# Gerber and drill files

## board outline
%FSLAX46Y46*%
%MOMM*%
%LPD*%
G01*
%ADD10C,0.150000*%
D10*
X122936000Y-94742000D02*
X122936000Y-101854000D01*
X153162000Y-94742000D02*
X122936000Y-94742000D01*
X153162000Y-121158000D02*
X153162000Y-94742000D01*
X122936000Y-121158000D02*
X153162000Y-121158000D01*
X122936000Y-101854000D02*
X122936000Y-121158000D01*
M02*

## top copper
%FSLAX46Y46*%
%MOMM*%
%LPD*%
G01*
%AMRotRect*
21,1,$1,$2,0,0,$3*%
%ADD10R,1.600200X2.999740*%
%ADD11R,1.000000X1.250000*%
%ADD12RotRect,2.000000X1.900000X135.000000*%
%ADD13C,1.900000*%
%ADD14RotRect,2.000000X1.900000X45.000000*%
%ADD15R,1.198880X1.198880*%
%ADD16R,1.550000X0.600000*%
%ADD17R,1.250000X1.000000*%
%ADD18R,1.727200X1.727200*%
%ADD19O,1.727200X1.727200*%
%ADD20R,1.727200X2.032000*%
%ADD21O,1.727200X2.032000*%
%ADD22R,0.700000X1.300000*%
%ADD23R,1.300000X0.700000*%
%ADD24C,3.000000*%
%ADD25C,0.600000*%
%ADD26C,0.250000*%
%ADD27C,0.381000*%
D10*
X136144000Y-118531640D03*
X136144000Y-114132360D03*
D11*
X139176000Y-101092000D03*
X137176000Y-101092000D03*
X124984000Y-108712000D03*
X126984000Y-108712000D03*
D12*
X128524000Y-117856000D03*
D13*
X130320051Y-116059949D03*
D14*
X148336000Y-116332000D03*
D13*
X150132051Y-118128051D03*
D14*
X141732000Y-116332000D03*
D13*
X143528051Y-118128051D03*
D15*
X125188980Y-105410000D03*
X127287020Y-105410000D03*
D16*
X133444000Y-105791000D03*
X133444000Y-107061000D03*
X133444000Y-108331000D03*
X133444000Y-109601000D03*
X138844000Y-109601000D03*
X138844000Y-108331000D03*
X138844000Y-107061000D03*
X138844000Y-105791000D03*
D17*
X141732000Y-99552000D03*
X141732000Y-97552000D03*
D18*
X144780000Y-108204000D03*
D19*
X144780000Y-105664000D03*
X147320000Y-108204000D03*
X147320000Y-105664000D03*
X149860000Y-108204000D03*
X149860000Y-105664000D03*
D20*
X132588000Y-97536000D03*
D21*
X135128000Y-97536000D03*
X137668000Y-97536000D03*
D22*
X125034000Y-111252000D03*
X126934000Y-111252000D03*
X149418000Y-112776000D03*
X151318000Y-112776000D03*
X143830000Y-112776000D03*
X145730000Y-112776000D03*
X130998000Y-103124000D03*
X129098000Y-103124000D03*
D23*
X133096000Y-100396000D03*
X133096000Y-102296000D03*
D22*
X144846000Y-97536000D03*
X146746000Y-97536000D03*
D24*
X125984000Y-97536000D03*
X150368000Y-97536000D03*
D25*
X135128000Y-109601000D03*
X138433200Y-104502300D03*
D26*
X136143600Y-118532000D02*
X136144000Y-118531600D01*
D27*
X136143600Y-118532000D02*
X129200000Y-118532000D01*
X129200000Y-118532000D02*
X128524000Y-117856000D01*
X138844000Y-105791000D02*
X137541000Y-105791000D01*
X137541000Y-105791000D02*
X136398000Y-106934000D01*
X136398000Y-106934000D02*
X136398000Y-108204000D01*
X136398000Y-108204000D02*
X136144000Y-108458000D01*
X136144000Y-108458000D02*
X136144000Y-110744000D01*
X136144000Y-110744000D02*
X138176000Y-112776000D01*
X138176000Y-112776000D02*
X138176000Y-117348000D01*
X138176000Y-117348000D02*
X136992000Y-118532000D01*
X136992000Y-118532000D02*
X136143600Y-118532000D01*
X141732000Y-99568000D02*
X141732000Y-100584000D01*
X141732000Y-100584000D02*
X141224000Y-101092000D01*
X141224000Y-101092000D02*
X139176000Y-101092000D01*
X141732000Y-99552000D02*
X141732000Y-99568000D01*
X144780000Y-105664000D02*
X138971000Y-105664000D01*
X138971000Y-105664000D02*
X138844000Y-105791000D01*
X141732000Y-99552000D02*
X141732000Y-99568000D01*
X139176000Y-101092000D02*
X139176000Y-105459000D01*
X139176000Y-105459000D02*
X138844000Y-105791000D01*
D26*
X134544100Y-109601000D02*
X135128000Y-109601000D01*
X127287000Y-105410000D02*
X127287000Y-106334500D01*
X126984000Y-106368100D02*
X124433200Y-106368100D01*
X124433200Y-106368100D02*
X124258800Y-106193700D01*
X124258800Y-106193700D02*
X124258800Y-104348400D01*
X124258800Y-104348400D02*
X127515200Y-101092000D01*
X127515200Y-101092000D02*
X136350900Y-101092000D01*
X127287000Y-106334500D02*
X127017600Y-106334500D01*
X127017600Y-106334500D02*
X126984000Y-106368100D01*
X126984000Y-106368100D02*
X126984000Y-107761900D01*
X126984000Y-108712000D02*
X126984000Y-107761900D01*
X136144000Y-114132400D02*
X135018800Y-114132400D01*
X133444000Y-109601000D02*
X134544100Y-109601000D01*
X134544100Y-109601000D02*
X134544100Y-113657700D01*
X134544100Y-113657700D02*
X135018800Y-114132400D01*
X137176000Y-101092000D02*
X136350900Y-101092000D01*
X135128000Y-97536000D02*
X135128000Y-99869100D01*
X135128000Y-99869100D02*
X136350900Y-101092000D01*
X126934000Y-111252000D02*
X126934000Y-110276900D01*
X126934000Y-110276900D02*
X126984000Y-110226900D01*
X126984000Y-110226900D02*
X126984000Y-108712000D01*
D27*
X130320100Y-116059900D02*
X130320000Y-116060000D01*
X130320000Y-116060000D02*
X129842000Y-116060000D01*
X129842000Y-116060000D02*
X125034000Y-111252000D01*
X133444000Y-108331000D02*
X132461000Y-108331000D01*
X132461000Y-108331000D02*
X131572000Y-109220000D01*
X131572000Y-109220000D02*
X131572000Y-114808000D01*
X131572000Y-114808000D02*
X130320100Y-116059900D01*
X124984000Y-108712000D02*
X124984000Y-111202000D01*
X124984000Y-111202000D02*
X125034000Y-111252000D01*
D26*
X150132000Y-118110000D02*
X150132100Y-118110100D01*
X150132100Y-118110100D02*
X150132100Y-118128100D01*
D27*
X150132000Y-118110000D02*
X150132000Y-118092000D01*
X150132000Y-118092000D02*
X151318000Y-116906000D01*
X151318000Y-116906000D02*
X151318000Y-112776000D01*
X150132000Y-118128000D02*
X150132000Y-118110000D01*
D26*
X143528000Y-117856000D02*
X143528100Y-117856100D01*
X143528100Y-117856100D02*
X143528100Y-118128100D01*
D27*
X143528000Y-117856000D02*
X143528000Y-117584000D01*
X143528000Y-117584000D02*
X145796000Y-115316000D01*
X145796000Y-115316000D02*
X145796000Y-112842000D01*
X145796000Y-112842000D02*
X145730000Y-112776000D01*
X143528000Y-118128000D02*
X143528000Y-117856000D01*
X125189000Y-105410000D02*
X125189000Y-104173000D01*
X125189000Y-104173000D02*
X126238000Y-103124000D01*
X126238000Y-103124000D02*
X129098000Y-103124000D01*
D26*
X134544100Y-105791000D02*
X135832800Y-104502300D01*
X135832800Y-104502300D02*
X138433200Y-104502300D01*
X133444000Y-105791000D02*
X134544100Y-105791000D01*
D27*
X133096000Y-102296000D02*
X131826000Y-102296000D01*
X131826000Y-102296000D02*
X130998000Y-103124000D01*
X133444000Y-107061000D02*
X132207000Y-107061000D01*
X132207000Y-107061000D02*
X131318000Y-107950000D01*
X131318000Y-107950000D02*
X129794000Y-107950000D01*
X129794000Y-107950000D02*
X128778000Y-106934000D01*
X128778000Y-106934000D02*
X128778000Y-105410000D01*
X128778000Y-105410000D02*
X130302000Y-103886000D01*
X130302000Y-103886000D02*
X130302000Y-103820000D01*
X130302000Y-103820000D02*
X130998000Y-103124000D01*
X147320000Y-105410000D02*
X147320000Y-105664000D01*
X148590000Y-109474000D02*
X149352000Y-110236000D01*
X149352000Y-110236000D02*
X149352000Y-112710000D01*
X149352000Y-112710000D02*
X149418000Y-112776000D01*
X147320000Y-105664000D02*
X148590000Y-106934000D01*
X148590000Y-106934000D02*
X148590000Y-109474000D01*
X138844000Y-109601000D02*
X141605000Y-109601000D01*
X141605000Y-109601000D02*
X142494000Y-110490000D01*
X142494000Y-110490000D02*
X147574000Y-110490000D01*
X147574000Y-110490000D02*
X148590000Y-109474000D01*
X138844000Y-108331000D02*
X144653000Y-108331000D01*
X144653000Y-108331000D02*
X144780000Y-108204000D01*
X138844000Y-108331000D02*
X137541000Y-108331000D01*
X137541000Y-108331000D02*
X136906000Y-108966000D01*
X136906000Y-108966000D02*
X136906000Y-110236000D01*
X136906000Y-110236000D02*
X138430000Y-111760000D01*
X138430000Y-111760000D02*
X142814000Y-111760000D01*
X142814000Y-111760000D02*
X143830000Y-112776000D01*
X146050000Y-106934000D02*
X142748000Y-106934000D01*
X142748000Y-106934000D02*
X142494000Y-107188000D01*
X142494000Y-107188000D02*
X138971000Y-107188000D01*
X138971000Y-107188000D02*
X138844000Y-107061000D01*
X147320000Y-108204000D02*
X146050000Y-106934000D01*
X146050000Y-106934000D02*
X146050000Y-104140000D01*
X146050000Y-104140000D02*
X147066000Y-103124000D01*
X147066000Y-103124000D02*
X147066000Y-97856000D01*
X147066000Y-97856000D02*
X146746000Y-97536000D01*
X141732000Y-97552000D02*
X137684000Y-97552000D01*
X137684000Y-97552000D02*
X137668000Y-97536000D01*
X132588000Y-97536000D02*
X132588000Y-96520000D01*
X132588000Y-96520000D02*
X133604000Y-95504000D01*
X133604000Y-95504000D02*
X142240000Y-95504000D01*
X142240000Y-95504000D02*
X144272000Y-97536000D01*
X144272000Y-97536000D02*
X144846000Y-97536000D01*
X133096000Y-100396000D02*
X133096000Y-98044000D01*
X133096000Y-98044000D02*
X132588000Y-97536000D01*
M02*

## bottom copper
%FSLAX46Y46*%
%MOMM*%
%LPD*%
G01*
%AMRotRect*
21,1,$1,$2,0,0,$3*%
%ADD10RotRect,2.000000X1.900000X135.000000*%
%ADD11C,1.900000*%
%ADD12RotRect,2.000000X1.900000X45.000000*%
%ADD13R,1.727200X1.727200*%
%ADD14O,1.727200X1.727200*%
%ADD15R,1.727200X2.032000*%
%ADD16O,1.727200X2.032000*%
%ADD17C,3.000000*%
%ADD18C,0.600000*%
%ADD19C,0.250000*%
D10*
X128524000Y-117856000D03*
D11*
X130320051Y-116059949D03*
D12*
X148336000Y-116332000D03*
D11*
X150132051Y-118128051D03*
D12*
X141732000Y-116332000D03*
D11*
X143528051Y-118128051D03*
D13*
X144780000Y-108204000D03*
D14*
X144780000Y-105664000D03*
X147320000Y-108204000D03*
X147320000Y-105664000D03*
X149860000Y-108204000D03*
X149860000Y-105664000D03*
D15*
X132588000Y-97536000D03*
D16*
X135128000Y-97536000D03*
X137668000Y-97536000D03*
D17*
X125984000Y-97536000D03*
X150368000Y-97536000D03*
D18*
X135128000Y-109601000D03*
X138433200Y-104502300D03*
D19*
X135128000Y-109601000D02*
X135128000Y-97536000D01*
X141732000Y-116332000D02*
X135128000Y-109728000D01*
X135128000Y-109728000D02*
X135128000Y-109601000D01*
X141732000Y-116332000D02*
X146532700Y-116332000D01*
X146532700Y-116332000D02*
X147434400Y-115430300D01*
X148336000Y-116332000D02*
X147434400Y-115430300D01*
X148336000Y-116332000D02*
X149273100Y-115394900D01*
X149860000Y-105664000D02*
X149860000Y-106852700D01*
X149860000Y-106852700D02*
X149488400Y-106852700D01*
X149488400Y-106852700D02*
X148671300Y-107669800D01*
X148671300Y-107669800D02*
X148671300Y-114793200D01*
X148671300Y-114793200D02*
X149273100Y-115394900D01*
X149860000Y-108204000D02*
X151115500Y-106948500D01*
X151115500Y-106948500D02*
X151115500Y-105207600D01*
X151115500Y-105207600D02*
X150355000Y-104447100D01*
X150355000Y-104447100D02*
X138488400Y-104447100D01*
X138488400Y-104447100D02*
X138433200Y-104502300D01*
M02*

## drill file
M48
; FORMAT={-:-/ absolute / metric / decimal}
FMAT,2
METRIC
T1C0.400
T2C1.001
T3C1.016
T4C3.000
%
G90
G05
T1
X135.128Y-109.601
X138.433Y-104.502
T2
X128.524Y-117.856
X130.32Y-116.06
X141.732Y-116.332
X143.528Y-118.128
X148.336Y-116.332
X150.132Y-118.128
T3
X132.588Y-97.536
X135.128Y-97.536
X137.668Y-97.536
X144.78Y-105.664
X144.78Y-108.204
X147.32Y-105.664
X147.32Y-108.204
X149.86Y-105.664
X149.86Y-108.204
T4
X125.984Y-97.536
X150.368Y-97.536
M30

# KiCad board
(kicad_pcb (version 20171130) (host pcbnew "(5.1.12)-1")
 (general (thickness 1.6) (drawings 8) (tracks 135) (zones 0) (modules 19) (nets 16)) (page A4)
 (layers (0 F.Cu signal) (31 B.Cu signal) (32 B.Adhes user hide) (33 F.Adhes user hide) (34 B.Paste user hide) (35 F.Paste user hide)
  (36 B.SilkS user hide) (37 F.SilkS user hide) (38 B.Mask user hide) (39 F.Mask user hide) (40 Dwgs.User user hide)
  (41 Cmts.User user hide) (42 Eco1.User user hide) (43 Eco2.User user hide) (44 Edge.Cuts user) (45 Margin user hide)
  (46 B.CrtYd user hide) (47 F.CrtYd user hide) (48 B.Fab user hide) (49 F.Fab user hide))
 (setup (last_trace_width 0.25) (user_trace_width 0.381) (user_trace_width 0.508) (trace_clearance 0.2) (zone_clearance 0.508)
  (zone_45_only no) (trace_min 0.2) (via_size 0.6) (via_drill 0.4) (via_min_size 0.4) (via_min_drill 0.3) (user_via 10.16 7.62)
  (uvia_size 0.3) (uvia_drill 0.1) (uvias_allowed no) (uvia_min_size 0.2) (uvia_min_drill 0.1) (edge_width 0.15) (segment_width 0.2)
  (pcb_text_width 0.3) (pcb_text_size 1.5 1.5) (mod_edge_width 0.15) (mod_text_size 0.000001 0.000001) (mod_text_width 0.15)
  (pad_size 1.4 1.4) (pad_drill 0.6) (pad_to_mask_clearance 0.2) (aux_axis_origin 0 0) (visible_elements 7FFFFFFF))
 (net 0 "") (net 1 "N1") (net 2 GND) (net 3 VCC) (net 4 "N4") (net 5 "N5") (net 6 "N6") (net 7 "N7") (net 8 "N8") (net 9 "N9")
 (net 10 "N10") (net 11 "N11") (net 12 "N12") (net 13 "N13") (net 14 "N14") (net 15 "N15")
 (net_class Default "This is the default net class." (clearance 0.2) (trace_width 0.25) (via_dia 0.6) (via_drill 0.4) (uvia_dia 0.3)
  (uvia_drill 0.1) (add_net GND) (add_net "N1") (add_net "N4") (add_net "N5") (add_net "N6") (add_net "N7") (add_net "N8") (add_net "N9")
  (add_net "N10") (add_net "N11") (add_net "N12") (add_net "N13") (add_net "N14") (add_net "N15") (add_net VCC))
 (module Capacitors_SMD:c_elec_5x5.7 (layer F.Cu) (at 136.144 116.332 270)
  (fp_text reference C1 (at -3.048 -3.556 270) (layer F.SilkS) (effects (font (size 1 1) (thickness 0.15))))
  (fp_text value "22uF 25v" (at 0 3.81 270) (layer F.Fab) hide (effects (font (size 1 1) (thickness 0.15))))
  (pad 1 smd rect (at 2.19964 0 270) (size 2.99974 1.6002) (layers F.Cu F.Paste F.Mask) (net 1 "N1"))
  (pad 2 smd rect (at -2.19964 0 270) (size 2.99974 1.6002) (layers F.Cu F.Paste F.Mask) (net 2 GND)))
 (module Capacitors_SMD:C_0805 (layer F.Cu) (at 138.176 101.092 180)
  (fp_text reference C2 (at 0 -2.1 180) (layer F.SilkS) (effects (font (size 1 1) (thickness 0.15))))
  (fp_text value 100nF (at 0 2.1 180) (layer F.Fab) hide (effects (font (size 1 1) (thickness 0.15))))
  (pad 1 smd rect (at -1 0 180) (size 1 1.25) (layers F.Cu F.Paste F.Mask) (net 1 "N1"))
  (pad 2 smd rect (at 1 0 180) (size 1 1.25) (layers F.Cu F.Paste F.Mask) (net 2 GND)))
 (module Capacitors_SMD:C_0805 (layer F.Cu) (at 125.984 108.712)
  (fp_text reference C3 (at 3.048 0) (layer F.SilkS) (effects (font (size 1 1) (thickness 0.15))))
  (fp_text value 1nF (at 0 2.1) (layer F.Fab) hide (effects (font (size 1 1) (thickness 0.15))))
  (pad 1 smd rect (at -1 0) (size 1 1.25) (layers F.Cu F.Paste F.Mask) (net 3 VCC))
  (pad 2 smd rect (at 1 0) (size 1 1.25) (layers F.Cu F.Paste F.Mask) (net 2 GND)))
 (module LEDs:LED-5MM (layer F.Cu) (at 128.524 117.856 45)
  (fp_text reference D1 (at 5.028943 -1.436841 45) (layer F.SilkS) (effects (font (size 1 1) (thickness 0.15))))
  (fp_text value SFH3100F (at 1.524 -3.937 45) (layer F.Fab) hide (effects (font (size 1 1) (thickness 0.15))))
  (pad 1 thru_hole rect (at 0 0 135) (size 2 1.9) (drill 1.00076) (layers *.Cu *.Mask F.SilkS) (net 1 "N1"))
  (pad 2 thru_hole circle (at 2.54 0 45) (size 1.9 1.9) (drill 1.00076) (layers *.Cu *.Mask F.SilkS) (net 3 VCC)))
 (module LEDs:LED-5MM (layer F.Cu) (at 148.336 116.332 315)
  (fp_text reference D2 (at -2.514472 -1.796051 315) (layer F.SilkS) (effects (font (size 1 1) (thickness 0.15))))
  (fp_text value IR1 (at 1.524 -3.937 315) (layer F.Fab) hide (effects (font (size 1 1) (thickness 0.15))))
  (pad 1 thru_hole rect (at 0 0 45) (size 2 1.9) (drill 1.00076) (layers *.Cu *.Mask F.SilkS) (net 2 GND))
  (pad 2 thru_hole circle (at 2.54 0 315) (size 1.9 1.9) (drill 1.00076) (layers *.Cu *.Mask F.SilkS) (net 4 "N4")))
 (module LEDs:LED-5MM (layer F.Cu) (at 141.732 116.332 315)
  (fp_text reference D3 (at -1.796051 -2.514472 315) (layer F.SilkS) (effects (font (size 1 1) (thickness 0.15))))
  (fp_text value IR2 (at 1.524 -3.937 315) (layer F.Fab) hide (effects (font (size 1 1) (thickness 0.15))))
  (pad 1 thru_hole rect (at 0 0 45) (size 2 1.9) (drill 1.00076) (layers *.Cu *.Mask F.SilkS) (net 2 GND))
  (pad 2 thru_hole circle (at 2.54 0 315) (size 1.9 1.9) (drill 1.00076) (layers *.Cu *.Mask F.SilkS) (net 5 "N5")))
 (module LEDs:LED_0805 (layer F.Cu) (at 126.238 105.41 180)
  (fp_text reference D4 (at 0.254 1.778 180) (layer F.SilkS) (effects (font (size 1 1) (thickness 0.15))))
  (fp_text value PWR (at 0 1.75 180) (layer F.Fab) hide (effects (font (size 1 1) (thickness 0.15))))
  (pad 2 smd rect (at 1.04902 0) (size 1.19888 1.19888) (layers F.Cu F.Paste F.Mask) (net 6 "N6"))
  (pad 1 smd rect (at -1.04902 0) (size 1.19888 1.19888) (layers F.Cu F.Paste F.Mask) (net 2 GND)))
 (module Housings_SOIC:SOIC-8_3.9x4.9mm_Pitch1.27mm (layer F.Cu) (at 136.144 107.696)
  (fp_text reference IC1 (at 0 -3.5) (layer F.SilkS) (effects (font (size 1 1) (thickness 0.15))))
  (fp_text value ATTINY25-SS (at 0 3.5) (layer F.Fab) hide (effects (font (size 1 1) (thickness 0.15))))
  (pad 1 smd rect (at -2.7 -1.905) (size 1.55 0.6) (layers F.Cu F.Paste F.Mask) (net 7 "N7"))
  (pad 2 smd rect (at -2.7 -0.635) (size 1.55 0.6) (layers F.Cu F.Paste F.Mask) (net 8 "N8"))
  (pad 3 smd rect (at -2.7 0.635) (size 1.55 0.6) (layers F.Cu F.Paste F.Mask) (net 3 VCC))
  (pad 4 smd rect (at -2.7 1.905) (size 1.55 0.6) (layers F.Cu F.Paste F.Mask) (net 2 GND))
  (pad 5 smd rect (at 2.7 1.905) (size 1.55 0.6) (layers F.Cu F.Paste F.Mask) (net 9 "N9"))
  (pad 6 smd rect (at 2.7 0.635) (size 1.55 0.6) (layers F.Cu F.Paste F.Mask) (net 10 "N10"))
  (pad 7 smd rect (at 2.7 -0.635) (size 1.55 0.6) (layers F.Cu F.Paste F.Mask) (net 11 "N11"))
  (pad 8 smd rect (at 2.7 -1.905) (size 1.55 0.6) (layers F.Cu F.Paste F.Mask) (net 1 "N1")))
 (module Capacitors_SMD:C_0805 (layer F.Cu) (at 141.732 98.552 90)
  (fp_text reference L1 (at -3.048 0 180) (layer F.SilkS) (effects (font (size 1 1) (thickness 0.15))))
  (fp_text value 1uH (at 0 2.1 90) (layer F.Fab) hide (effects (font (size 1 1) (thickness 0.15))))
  (pad 1 smd rect (at -1 0 90) (size 1 1.25) (layers F.Cu F.Paste F.Mask) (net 1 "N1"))
  (pad 2 smd rect (at 1 0 90) (size 1 1.25) (layers F.Cu F.Paste F.Mask) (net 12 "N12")))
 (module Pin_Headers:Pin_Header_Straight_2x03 (layer F.Cu) (at 144.78 108.204 90)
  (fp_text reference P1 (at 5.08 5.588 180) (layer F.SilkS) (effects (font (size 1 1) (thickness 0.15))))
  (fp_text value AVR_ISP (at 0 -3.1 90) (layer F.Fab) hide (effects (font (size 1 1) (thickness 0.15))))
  (pad 1 thru_hole rect (at 0 0 90) (size 1.7272 1.7272) (drill 1.016) (layers *.Cu *.Mask F.SilkS) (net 10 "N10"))
  (pad 2 thru_hole oval (at 2.54 0 90) (size 1.7272 1.7272) (drill 1.016) (layers *.Cu *.Mask F.SilkS) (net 1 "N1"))
  (pad 3 thru_hole oval (at 0 2.54 90) (size 1.7272 1.7272) (drill 1.016) (layers *.Cu *.Mask F.SilkS) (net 11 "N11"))
  (pad 4 thru_hole oval (at 2.54 2.54 90) (size 1.7272 1.7272) (drill 1.016) (layers *.Cu *.Mask F.SilkS) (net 9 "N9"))
  (pad 5 thru_hole oval (at 0 5.08 90) (size 1.7272 1.7272) (drill 1.016) (layers *.Cu *.Mask F.SilkS) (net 7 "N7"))
  (pad 6 thru_hole oval (at 2.54 5.08 90) (size 1.7272 1.7272) (drill 1.016) (layers *.Cu *.Mask F.SilkS) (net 2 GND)))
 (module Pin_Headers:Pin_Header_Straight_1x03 (layer F.Cu) (at 132.588 97.536 90)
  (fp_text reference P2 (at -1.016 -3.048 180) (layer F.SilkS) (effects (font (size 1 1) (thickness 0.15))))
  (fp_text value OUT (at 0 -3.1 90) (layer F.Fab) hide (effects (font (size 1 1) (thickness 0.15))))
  (pad 1 thru_hole rect (at 0 0 90) (size 2.032 1.7272) (drill 1.016) (layers *.Cu *.Mask F.SilkS) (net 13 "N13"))
  (pad 2 thru_hole oval (at 0 2.54 90) (size 2.032 1.7272) (drill 1.016) (layers *.Cu *.Mask F.SilkS) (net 2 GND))
  (pad 3 thru_hole oval (at 0 5.08 90) (size 2.032 1.7272) (drill 1.016) (layers *.Cu *.Mask F.SilkS) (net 12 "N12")))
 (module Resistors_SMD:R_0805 (layer F.Cu) (at 125.984 111.252)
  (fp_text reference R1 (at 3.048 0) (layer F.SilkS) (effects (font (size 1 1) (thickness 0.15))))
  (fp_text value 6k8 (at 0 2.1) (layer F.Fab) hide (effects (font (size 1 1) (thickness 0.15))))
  (pad 1 smd rect (at -0.95 0) (size 0.7 1.3) (layers F.Cu F.Paste F.Mask) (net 3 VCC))
  (pad 2 smd rect (at 0.95 0) (size 0.7 1.3) (layers F.Cu F.Paste F.Mask) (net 2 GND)))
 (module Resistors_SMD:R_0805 (layer F.Cu) (at 150.368 112.776)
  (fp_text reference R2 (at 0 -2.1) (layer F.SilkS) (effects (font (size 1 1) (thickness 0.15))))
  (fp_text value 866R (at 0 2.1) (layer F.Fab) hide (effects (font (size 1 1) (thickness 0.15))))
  (pad 1 smd rect (at -0.95 0) (size 0.7 1.3) (layers F.Cu F.Paste F.Mask) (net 9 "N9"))
  (pad 2 smd rect (at 0.95 0) (size 0.7 1.3) (layers F.Cu F.Paste F.Mask) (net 4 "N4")))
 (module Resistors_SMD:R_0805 (layer F.Cu) (at 144.78 112.776)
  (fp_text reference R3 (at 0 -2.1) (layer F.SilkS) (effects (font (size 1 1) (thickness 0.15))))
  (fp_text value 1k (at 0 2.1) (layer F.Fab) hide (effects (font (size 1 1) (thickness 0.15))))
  (pad 1 smd rect (at -0.95 0) (size 0.7 1.3) (layers F.Cu F.Paste F.Mask) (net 10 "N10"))
  (pad 2 smd rect (at 0.95 0) (size 0.7 1.3) (layers F.Cu F.Paste F.Mask) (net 5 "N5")))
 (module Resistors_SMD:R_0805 (layer F.Cu) (at 130.048 103.124 180)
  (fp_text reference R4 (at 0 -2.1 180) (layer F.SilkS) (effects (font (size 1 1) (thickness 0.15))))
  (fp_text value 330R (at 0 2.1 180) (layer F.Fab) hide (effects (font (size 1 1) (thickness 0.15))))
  (pad 1 smd rect (at -0.95 0 180) (size 0.7 1.3) (layers F.Cu F.Paste F.Mask) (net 8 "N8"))
  (pad 2 smd rect (at 0.95 0 180) (size 0.7 1.3) (layers F.Cu F.Paste F.Mask) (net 6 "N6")))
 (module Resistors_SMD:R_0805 (layer F.Cu) (at 133.096 101.346 270)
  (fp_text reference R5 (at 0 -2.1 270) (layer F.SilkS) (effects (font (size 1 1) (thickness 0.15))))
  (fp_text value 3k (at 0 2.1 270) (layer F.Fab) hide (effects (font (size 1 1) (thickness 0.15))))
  (pad 1 smd rect (at -0.95 0 270) (size 0.7 1.3) (layers F.Cu F.Paste F.Mask) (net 13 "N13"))
  (pad 2 smd rect (at 0.95 0 270) (size 0.7 1.3) (layers F.Cu F.Paste F.Mask) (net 8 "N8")))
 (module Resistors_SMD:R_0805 (layer F.Cu) (at 145.796 97.536)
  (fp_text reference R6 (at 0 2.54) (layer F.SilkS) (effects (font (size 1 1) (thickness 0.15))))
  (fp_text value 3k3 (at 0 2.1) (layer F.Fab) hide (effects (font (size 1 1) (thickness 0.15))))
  (pad 1 smd rect (at -0.95 0) (size 0.7 1.3) (layers F.Cu F.Paste F.Mask) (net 13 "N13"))
  (pad 2 smd rect (at 0.95 0) (size 0.7 1.3) (layers F.Cu F.Paste F.Mask) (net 11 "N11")))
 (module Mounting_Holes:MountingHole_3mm (layer F.Cu) (at 125.984 97.536)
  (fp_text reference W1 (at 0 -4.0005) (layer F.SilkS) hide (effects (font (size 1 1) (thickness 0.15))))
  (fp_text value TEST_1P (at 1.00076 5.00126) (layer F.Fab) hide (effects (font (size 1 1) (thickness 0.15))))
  (pad 1 thru_hole circle (at 0 0) (size 3 3) (drill 3) (layers *.Cu *.Mask) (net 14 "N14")))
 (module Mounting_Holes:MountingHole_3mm (layer F.Cu) (at 150.368 97.536)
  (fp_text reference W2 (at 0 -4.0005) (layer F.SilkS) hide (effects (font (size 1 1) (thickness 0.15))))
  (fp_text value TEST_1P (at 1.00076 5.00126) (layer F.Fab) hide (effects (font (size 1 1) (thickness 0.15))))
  (pad 1 thru_hole circle (at 0 0) (size 3 3) (drill 3) (layers *.Cu *.Mask) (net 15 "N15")))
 (gr_line (start 122.936 94.742) (end 122.936 101.854) (angle 90) (layer Edge.Cuts) (width 0.15))
 (gr_line (start 153.162 94.742) (end 122.936 94.742) (angle 90) (layer Edge.Cuts) (width 0.15))
 (gr_line (start 153.162 121.158) (end 153.162 94.742) (angle 90) (layer Edge.Cuts) (width 0.15))
 (gr_line (start 122.936 121.158) (end 153.162 121.158) (angle 90) (layer Edge.Cuts) (width 0.15))
 (gr_line (start 122.936 101.854) (end 122.936 121.158) (angle 90) (layer Edge.Cuts) (width 0.15))
 (segment (start 136.1436 118.532) (end 136.144 118.5316) (width 0.25) (layer F.Cu) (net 1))
 (segment (start 136.1436 118.532) (end 129.2 118.532) (width 0.381) (layer F.Cu) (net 1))
 (segment (start 129.2 118.532) (end 128.524 117.856) (width 0.381) (layer F.Cu) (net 1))
 (segment (start 138.844 105.791) (end 137.541 105.791) (width 0.381) (layer F.Cu) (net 1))
 (segment (start 137.541 105.791) (end 136.398 106.934) (width 0.381) (layer F.Cu) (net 1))
 (segment (start 136.398 106.934) (end 136.398 108.204) (width 0.381) (layer F.Cu) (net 1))
 (segment (start 136.398 108.204) (end 136.144 108.458) (width 0.381) (layer F.Cu) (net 1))
 (segment (start 136.144 108.458) (end 136.144 110.744) (width 0.381) (layer F.Cu) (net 1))
 (segment (start 136.144 110.744) (end 138.176 112.776) (width 0.381) (layer F.Cu) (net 1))
 (segment (start 138.176 112.776) (end 138.176 117.348) (width 0.381) (layer F.Cu) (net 1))
 (segment (start 138.176 117.348) (end 136.992 118.532) (width 0.381) (layer F.Cu) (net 1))
 (segment (start 136.992 118.532) (end 136.1436 118.532) (width 0.381) (layer F.Cu) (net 1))
 (segment (start 141.732 99.568) (end 141.732 100.584) (width 0.381) (layer F.Cu) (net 1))
 (segment (start 141.732 100.584) (end 141.224 101.092) (width 0.381) (layer F.Cu) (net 1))
 (segment (start 141.224 101.092) (end 139.176 101.092) (width 0.381) (layer F.Cu) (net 1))
 (segment (start 141.732 99.552) (end 141.732 99.568) (width 0.381) (layer F.Cu) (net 1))
 (segment (start 144.78 105.664) (end 138.971 105.664) (width 0.381) (layer F.Cu) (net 1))
 (segment (start 138.971 105.664) (end 138.844 105.791) (width 0.381) (layer F.Cu) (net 1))
 (segment (start 141.732 99.552) (end 141.732 99.568) (width 0.381) (layer F.Cu) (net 1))
 (segment (start 139.176 101.092) (end 139.176 105.459) (width 0.381) (layer F.Cu) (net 1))
 (segment (start 139.176 105.459) (end 138.844 105.791) (width 0.381) (layer F.Cu) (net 1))
 (segment (start 134.5441 109.601) (end 135.128 109.601) (width 0.25) (layer F.Cu) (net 2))
 (segment (start 135.128 109.601) (end 135.128 97.536) (width 0.25) (layer B.Cu) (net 2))
 (segment (start 141.732 116.332) (end 135.128 109.728) (width 0.25) (layer B.Cu) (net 2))
 (segment (start 135.128 109.728) (end 135.128 109.601) (width 0.25) (layer B.Cu) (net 2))
 (segment (start 127.287 105.41) (end 127.287 106.3345) (width 0.25) (layer F.Cu) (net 2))
 (segment (start 126.984 106.3681) (end 124.4332 106.3681) (width 0.25) (layer F.Cu) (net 2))
 (segment (start 124.4332 106.3681) (end 124.2588 106.1937) (width 0.25) (layer F.Cu) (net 2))
 (segment (start 124.2588 106.1937) (end 124.2588 104.3484) (width 0.25) (layer F.Cu) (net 2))
 (segment (start 124.2588 104.3484) (end 127.5152 101.092) (width 0.25) (layer F.Cu) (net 2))
 (segment (start 127.5152 101.092) (end 136.3509 101.092) (width 0.25) (layer F.Cu) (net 2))
 (segment (start 127.287 106.3345) (end 127.0176 106.3345) (width 0.25) (layer F.Cu) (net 2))
 (segment (start 127.0176 106.3345) (end 126.984 106.3681) (width 0.25) (layer F.Cu) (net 2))
 (segment (start 126.984 106.3681) (end 126.984 107.7619) (width 0.25) (layer F.Cu) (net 2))
 (segment (start 141.732 116.332) (end 146.5327 116.332) (width 0.25) (layer B.Cu) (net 2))
 (segment (start 146.5327 116.332) (end 147.4344 115.4303) (width 0.25) (layer B.Cu) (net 2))
 (segment (start 148.336 116.332) (end 147.4344 115.4303) (width 0.25) (layer B.Cu) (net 2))
 (segment (start 126.984 108.712) (end 126.984 107.7619) (width 0.25) (layer F.Cu) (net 2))
 (segment (start 136.144 114.1324) (end 135.0188 114.1324) (width 0.25) (layer F.Cu) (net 2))
 (segment (start 133.444 109.601) (end 134.5441 109.601) (width 0.25) (layer F.Cu) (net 2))
 (segment (start 134.5441 109.601) (end 134.5441 113.6577) (width 0.25) (layer F.Cu) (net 2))
 (segment (start 134.5441 113.6577) (end 135.0188 114.1324) (width 0.25) (layer F.Cu) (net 2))
 (segment (start 148.336 116.332) (end 149.2731 115.3949) (width 0.25) (layer B.Cu) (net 2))
 (segment (start 149.86 105.664) (end 149.86 106.8527) (width 0.25) (layer B.Cu) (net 2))
 (segment (start 149.86 106.8527) (end 149.4884 106.8527) (width 0.25) (layer B.Cu) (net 2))
 (segment (start 149.4884 106.8527) (end 148.6713 107.6698) (width 0.25) (layer B.Cu) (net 2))
 (segment (start 148.6713 107.6698) (end 148.6713 114.7932) (width 0.25) (layer B.Cu) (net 2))
 (segment (start 148.6713 114.7932) (end 149.2731 115.3949) (width 0.25) (layer B.Cu) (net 2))
 (segment (start 137.176 101.092) (end 136.3509 101.092) (width 0.25) (layer F.Cu) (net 2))
 (segment (start 135.128 97.536) (end 135.128 99.8691) (width 0.25) (layer F.Cu) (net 2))
 (segment (start 135.128 99.8691) (end 136.3509 101.092) (width 0.25) (layer F.Cu) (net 2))
 (segment (start 126.934 111.252) (end 126.934 110.2769) (width 0.25) (layer F.Cu) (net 2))
 (segment (start 126.934 110.2769) (end 126.984 110.2269) (width 0.25) (layer F.Cu) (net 2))
 (segment (start 126.984 110.2269) (end 126.984 108.712) (width 0.25) (layer F.Cu) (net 2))
 (via (at 135.128 109.601) (size 0.6) (layers F.Cu B.Cu) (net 2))
 (segment (start 130.3201 116.0599) (end 130.32 116.06) (width 0.381) (layer F.Cu) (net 3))
 (segment (start 130.32 116.06) (end 129.842 116.06) (width 0.381) (layer F.Cu) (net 3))
 (segment (start 129.842 116.06) (end 125.034 111.252) (width 0.381) (layer F.Cu) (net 3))
 (segment (start 133.444 108.331) (end 132.461 108.331) (width 0.381) (layer F.Cu) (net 3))
 (segment (start 132.461 108.331) (end 131.572 109.22) (width 0.381) (layer F.Cu) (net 3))
 (segment (start 131.572 109.22) (end 131.572 114.808) (width 0.381) (layer F.Cu) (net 3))
 (segment (start 131.572 114.808) (end 130.3201 116.0599) (width 0.381) (layer F.Cu) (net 3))
 (segment (start 124.984 108.712) (end 124.984 111.202) (width 0.381) (layer F.Cu) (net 3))
 (segment (start 124.984 111.202) (end 125.034 111.252) (width 0.381) (layer F.Cu) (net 3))
 (segment (start 150.132 118.11) (end 150.1321 118.1101) (width 0.25) (layer F.Cu) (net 4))
 (segment (start 150.1321 118.1101) (end 150.1321 118.1281) (width 0.25) (layer F.Cu) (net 4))
 (segment (start 150.132 118.11) (end 150.132 118.092) (width 0.381) (layer F.Cu) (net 4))
 (segment (start 150.132 118.092) (end 151.318 116.906) (width 0.381) (layer F.Cu) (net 4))
 (segment (start 151.318 116.906) (end 151.318 112.776) (width 0.381) (layer F.Cu) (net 4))
 (segment (start 150.132 118.128) (end 150.132 118.11) (width 0.381) (layer F.Cu) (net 4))
 (segment (start 143.528 117.856) (end 143.5281 117.8561) (width 0.25) (layer F.Cu) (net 5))
 (segment (start 143.5281 117.8561) (end 143.5281 118.1281) (width 0.25) (layer F.Cu) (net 5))
 (segment (start 143.528 117.856) (end 143.528 117.584) (width 0.381) (layer F.Cu) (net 5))
 (segment (start 143.528 117.584) (end 145.796 115.316) (width 0.381) (layer F.Cu) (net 5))
 (segment (start 145.796 115.316) (end 145.796 112.842) (width 0.381) (layer F.Cu) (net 5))
 (segment (start 145.796 112.842) (end 145.73 112.776) (width 0.381) (layer F.Cu) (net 5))
 (segment (start 143.528 118.128) (end 143.528 117.856) (width 0.381) (layer F.Cu) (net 5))
 (segment (start 125.189 105.41) (end 125.189 104.173) (width 0.381) (layer F.Cu) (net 6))
 (segment (start 125.189 104.173) (end 126.238 103.124) (width 0.381) (layer F.Cu) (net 6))
 (segment (start 126.238 103.124) (end 129.098 103.124) (width 0.381) (layer F.Cu) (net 6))
 (segment (start 134.5441 105.791) (end 135.8328 104.5023) (width 0.25) (layer F.Cu) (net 7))
 (segment (start 135.8328 104.5023) (end 138.4332 104.5023) (width 0.25) (layer F.Cu) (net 7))
 (segment (start 149.86 108.204) (end 151.1155 106.9485) (width 0.25) (layer B.Cu) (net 7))
 (segment (start 151.1155 106.9485) (end 151.1155 105.2076) (width 0.25) (layer B.Cu) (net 7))
 (segment (start 151.1155 105.2076) (end 150.355 104.4471) (width 0.25) (layer B.Cu) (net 7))
 (segment (start 150.355 104.4471) (end 138.4884 104.4471) (width 0.25) (layer B.Cu) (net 7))
 (segment (start 138.4884 104.4471) (end 138.4332 104.5023) (width 0.25) (layer B.Cu) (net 7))
 (segment (start 133.444 105.791) (end 134.5441 105.791) (width 0.25) (layer F.Cu) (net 7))
 (via (at 138.4332 104.5023) (size 0.6) (layers F.Cu B.Cu) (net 7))
 (segment (start 133.096 102.296) (end 131.826 102.296) (width 0.381) (layer F.Cu) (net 8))
 (segment (start 131.826 102.296) (end 130.998 103.124) (width 0.381) (layer F.Cu) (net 8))
 (segment (start 133.444 107.061) (end 132.207 107.061) (width 0.381) (layer F.Cu) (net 8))
 (segment (start 132.207 107.061) (end 131.318 107.95) (width 0.381) (layer F.Cu) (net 8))
 (segment (start 131.318 107.95) (end 129.794 107.95) (width 0.381) (layer F.Cu) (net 8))
 (segment (start 129.794 107.95) (end 128.778 106.934) (width 0.381) (layer F.Cu) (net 8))
 (segment (start 128.778 106.934) (end 128.778 105.41) (width 0.381) (layer F.Cu) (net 8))
 (segment (start 128.778 105.41) (end 130.302 103.886) (width 0.381) (layer F.Cu) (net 8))
 (segment (start 130.302 103.886) (end 130.302 103.82) (width 0.381) (layer F.Cu) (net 8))
 (segment (start 130.302 103.82) (end 130.998 103.124) (width 0.381) (layer F.Cu) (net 8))
 (segment (start 147.32 105.41) (end 147.32 105.664) (width 0.381) (layer F.Cu) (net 9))
 (segment (start 148.59 109.474) (end 149.352 110.236) (width 0.381) (layer F.Cu) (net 9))
 (segment (start 149.352 110.236) (end 149.352 112.71) (width 0.381) (layer F.Cu) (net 9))
 (segment (start 149.352 112.71) (end 149.418 112.776) (width 0.381) (layer F.Cu) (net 9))
 (segment (start 147.32 105.664) (end 148.59 106.934) (width 0.381) (layer F.Cu) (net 9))
 (segment (start 148.59 106.934) (end 148.59 109.474) (width 0.381) (layer F.Cu) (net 9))
 (segment (start 138.844 109.601) (end 141.605 109.601) (width 0.381) (layer F.Cu) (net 9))
 (segment (start 141.605 109.601) (end 142.494 110.49) (width 0.381) (layer F.Cu) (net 9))
 (segment (start 142.494 110.49) (end 147.574 110.49) (width 0.381) (layer F.Cu) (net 9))
 (segment (start 147.574 110.49) (end 148.59 109.474) (width 0.381) (layer F.Cu) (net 9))
 (segment (start 138.844 108.331) (end 144.653 108.331) (width 0.381) (layer F.Cu) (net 10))
 (segment (start 144.653 108.331) (end 144.78 108.204) (width 0.381) (layer F.Cu) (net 10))
 (segment (start 138.844 108.331) (end 137.541 108.331) (width 0.381) (layer F.Cu) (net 10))
 (segment (start 137.541 108.331) (end 136.906 108.966) (width 0.381) (layer F.Cu) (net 10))
 (segment (start 136.906 108.966) (end 136.906 110.236) (width 0.381) (layer F.Cu) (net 10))
 (segment (start 136.906 110.236) (end 138.43 111.76) (width 0.381) (layer F.Cu) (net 10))
 (segment (start 138.43 111.76) (end 142.814 111.76) (width 0.381) (layer F.Cu) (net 10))
 (segment (start 142.814 111.76) (end 143.83 112.776) (width 0.381) (layer F.Cu) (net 10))
 (segment (start 146.05 106.934) (end 142.748 106.934) (width 0.381) (layer F.Cu) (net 11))
 (segment (start 142.748 106.934) (end 142.494 107.188) (width 0.381) (layer F.Cu) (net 11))
 (segment (start 142.494 107.188) (end 138.971 107.188) (width 0.381) (layer F.Cu) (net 11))
 (segment (start 138.971 107.188) (end 138.844 107.061) (width 0.381) (layer F.Cu) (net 11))
 (segment (start 147.32 108.204) (end 146.05 106.934) (width 0.381) (layer F.Cu) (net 11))
 (segment (start 146.05 106.934) (end 146.05 104.14) (width 0.381) (layer F.Cu) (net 11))
 (segment (start 146.05 104.14) (end 147.066 103.124) (width 0.381) (layer F.Cu) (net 11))
 (segment (start 147.066 103.124) (end 147.066 97.856) (width 0.381) (layer F.Cu) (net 11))
 (segment (start 147.066 97.856) (end 146.746 97.536) (width 0.381) (layer F.Cu) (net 11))
 (segment (start 141.732 97.552) (end 137.684 97.552) (width 0.381) (layer F.Cu) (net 12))
 (segment (start 137.684 97.552) (end 137.668 97.536) (width 0.381) (layer F.Cu) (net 12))
 (segment (start 132.588 97.536) (end 132.588 96.52) (width 0.381) (layer F.Cu) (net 13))
 (segment (start 132.588 96.52) (end 133.604 95.504) (width 0.381) (layer F.Cu) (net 13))
 (segment (start 133.604 95.504) (end 142.24 95.504) (width 0.381) (layer F.Cu) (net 13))
 (segment (start 142.24 95.504) (end 144.272 97.536) (width 0.381) (layer F.Cu) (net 13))
 (segment (start 144.272 97.536) (end 144.846 97.536) (width 0.381) (layer F.Cu) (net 13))
 (segment (start 133.096 100.396) (end 133.096 98.044) (width 0.381) (layer F.Cu) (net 13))
 (segment (start 133.096 98.044) (end 132.588 97.536) (width 0.381) (layer F.Cu) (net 13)))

